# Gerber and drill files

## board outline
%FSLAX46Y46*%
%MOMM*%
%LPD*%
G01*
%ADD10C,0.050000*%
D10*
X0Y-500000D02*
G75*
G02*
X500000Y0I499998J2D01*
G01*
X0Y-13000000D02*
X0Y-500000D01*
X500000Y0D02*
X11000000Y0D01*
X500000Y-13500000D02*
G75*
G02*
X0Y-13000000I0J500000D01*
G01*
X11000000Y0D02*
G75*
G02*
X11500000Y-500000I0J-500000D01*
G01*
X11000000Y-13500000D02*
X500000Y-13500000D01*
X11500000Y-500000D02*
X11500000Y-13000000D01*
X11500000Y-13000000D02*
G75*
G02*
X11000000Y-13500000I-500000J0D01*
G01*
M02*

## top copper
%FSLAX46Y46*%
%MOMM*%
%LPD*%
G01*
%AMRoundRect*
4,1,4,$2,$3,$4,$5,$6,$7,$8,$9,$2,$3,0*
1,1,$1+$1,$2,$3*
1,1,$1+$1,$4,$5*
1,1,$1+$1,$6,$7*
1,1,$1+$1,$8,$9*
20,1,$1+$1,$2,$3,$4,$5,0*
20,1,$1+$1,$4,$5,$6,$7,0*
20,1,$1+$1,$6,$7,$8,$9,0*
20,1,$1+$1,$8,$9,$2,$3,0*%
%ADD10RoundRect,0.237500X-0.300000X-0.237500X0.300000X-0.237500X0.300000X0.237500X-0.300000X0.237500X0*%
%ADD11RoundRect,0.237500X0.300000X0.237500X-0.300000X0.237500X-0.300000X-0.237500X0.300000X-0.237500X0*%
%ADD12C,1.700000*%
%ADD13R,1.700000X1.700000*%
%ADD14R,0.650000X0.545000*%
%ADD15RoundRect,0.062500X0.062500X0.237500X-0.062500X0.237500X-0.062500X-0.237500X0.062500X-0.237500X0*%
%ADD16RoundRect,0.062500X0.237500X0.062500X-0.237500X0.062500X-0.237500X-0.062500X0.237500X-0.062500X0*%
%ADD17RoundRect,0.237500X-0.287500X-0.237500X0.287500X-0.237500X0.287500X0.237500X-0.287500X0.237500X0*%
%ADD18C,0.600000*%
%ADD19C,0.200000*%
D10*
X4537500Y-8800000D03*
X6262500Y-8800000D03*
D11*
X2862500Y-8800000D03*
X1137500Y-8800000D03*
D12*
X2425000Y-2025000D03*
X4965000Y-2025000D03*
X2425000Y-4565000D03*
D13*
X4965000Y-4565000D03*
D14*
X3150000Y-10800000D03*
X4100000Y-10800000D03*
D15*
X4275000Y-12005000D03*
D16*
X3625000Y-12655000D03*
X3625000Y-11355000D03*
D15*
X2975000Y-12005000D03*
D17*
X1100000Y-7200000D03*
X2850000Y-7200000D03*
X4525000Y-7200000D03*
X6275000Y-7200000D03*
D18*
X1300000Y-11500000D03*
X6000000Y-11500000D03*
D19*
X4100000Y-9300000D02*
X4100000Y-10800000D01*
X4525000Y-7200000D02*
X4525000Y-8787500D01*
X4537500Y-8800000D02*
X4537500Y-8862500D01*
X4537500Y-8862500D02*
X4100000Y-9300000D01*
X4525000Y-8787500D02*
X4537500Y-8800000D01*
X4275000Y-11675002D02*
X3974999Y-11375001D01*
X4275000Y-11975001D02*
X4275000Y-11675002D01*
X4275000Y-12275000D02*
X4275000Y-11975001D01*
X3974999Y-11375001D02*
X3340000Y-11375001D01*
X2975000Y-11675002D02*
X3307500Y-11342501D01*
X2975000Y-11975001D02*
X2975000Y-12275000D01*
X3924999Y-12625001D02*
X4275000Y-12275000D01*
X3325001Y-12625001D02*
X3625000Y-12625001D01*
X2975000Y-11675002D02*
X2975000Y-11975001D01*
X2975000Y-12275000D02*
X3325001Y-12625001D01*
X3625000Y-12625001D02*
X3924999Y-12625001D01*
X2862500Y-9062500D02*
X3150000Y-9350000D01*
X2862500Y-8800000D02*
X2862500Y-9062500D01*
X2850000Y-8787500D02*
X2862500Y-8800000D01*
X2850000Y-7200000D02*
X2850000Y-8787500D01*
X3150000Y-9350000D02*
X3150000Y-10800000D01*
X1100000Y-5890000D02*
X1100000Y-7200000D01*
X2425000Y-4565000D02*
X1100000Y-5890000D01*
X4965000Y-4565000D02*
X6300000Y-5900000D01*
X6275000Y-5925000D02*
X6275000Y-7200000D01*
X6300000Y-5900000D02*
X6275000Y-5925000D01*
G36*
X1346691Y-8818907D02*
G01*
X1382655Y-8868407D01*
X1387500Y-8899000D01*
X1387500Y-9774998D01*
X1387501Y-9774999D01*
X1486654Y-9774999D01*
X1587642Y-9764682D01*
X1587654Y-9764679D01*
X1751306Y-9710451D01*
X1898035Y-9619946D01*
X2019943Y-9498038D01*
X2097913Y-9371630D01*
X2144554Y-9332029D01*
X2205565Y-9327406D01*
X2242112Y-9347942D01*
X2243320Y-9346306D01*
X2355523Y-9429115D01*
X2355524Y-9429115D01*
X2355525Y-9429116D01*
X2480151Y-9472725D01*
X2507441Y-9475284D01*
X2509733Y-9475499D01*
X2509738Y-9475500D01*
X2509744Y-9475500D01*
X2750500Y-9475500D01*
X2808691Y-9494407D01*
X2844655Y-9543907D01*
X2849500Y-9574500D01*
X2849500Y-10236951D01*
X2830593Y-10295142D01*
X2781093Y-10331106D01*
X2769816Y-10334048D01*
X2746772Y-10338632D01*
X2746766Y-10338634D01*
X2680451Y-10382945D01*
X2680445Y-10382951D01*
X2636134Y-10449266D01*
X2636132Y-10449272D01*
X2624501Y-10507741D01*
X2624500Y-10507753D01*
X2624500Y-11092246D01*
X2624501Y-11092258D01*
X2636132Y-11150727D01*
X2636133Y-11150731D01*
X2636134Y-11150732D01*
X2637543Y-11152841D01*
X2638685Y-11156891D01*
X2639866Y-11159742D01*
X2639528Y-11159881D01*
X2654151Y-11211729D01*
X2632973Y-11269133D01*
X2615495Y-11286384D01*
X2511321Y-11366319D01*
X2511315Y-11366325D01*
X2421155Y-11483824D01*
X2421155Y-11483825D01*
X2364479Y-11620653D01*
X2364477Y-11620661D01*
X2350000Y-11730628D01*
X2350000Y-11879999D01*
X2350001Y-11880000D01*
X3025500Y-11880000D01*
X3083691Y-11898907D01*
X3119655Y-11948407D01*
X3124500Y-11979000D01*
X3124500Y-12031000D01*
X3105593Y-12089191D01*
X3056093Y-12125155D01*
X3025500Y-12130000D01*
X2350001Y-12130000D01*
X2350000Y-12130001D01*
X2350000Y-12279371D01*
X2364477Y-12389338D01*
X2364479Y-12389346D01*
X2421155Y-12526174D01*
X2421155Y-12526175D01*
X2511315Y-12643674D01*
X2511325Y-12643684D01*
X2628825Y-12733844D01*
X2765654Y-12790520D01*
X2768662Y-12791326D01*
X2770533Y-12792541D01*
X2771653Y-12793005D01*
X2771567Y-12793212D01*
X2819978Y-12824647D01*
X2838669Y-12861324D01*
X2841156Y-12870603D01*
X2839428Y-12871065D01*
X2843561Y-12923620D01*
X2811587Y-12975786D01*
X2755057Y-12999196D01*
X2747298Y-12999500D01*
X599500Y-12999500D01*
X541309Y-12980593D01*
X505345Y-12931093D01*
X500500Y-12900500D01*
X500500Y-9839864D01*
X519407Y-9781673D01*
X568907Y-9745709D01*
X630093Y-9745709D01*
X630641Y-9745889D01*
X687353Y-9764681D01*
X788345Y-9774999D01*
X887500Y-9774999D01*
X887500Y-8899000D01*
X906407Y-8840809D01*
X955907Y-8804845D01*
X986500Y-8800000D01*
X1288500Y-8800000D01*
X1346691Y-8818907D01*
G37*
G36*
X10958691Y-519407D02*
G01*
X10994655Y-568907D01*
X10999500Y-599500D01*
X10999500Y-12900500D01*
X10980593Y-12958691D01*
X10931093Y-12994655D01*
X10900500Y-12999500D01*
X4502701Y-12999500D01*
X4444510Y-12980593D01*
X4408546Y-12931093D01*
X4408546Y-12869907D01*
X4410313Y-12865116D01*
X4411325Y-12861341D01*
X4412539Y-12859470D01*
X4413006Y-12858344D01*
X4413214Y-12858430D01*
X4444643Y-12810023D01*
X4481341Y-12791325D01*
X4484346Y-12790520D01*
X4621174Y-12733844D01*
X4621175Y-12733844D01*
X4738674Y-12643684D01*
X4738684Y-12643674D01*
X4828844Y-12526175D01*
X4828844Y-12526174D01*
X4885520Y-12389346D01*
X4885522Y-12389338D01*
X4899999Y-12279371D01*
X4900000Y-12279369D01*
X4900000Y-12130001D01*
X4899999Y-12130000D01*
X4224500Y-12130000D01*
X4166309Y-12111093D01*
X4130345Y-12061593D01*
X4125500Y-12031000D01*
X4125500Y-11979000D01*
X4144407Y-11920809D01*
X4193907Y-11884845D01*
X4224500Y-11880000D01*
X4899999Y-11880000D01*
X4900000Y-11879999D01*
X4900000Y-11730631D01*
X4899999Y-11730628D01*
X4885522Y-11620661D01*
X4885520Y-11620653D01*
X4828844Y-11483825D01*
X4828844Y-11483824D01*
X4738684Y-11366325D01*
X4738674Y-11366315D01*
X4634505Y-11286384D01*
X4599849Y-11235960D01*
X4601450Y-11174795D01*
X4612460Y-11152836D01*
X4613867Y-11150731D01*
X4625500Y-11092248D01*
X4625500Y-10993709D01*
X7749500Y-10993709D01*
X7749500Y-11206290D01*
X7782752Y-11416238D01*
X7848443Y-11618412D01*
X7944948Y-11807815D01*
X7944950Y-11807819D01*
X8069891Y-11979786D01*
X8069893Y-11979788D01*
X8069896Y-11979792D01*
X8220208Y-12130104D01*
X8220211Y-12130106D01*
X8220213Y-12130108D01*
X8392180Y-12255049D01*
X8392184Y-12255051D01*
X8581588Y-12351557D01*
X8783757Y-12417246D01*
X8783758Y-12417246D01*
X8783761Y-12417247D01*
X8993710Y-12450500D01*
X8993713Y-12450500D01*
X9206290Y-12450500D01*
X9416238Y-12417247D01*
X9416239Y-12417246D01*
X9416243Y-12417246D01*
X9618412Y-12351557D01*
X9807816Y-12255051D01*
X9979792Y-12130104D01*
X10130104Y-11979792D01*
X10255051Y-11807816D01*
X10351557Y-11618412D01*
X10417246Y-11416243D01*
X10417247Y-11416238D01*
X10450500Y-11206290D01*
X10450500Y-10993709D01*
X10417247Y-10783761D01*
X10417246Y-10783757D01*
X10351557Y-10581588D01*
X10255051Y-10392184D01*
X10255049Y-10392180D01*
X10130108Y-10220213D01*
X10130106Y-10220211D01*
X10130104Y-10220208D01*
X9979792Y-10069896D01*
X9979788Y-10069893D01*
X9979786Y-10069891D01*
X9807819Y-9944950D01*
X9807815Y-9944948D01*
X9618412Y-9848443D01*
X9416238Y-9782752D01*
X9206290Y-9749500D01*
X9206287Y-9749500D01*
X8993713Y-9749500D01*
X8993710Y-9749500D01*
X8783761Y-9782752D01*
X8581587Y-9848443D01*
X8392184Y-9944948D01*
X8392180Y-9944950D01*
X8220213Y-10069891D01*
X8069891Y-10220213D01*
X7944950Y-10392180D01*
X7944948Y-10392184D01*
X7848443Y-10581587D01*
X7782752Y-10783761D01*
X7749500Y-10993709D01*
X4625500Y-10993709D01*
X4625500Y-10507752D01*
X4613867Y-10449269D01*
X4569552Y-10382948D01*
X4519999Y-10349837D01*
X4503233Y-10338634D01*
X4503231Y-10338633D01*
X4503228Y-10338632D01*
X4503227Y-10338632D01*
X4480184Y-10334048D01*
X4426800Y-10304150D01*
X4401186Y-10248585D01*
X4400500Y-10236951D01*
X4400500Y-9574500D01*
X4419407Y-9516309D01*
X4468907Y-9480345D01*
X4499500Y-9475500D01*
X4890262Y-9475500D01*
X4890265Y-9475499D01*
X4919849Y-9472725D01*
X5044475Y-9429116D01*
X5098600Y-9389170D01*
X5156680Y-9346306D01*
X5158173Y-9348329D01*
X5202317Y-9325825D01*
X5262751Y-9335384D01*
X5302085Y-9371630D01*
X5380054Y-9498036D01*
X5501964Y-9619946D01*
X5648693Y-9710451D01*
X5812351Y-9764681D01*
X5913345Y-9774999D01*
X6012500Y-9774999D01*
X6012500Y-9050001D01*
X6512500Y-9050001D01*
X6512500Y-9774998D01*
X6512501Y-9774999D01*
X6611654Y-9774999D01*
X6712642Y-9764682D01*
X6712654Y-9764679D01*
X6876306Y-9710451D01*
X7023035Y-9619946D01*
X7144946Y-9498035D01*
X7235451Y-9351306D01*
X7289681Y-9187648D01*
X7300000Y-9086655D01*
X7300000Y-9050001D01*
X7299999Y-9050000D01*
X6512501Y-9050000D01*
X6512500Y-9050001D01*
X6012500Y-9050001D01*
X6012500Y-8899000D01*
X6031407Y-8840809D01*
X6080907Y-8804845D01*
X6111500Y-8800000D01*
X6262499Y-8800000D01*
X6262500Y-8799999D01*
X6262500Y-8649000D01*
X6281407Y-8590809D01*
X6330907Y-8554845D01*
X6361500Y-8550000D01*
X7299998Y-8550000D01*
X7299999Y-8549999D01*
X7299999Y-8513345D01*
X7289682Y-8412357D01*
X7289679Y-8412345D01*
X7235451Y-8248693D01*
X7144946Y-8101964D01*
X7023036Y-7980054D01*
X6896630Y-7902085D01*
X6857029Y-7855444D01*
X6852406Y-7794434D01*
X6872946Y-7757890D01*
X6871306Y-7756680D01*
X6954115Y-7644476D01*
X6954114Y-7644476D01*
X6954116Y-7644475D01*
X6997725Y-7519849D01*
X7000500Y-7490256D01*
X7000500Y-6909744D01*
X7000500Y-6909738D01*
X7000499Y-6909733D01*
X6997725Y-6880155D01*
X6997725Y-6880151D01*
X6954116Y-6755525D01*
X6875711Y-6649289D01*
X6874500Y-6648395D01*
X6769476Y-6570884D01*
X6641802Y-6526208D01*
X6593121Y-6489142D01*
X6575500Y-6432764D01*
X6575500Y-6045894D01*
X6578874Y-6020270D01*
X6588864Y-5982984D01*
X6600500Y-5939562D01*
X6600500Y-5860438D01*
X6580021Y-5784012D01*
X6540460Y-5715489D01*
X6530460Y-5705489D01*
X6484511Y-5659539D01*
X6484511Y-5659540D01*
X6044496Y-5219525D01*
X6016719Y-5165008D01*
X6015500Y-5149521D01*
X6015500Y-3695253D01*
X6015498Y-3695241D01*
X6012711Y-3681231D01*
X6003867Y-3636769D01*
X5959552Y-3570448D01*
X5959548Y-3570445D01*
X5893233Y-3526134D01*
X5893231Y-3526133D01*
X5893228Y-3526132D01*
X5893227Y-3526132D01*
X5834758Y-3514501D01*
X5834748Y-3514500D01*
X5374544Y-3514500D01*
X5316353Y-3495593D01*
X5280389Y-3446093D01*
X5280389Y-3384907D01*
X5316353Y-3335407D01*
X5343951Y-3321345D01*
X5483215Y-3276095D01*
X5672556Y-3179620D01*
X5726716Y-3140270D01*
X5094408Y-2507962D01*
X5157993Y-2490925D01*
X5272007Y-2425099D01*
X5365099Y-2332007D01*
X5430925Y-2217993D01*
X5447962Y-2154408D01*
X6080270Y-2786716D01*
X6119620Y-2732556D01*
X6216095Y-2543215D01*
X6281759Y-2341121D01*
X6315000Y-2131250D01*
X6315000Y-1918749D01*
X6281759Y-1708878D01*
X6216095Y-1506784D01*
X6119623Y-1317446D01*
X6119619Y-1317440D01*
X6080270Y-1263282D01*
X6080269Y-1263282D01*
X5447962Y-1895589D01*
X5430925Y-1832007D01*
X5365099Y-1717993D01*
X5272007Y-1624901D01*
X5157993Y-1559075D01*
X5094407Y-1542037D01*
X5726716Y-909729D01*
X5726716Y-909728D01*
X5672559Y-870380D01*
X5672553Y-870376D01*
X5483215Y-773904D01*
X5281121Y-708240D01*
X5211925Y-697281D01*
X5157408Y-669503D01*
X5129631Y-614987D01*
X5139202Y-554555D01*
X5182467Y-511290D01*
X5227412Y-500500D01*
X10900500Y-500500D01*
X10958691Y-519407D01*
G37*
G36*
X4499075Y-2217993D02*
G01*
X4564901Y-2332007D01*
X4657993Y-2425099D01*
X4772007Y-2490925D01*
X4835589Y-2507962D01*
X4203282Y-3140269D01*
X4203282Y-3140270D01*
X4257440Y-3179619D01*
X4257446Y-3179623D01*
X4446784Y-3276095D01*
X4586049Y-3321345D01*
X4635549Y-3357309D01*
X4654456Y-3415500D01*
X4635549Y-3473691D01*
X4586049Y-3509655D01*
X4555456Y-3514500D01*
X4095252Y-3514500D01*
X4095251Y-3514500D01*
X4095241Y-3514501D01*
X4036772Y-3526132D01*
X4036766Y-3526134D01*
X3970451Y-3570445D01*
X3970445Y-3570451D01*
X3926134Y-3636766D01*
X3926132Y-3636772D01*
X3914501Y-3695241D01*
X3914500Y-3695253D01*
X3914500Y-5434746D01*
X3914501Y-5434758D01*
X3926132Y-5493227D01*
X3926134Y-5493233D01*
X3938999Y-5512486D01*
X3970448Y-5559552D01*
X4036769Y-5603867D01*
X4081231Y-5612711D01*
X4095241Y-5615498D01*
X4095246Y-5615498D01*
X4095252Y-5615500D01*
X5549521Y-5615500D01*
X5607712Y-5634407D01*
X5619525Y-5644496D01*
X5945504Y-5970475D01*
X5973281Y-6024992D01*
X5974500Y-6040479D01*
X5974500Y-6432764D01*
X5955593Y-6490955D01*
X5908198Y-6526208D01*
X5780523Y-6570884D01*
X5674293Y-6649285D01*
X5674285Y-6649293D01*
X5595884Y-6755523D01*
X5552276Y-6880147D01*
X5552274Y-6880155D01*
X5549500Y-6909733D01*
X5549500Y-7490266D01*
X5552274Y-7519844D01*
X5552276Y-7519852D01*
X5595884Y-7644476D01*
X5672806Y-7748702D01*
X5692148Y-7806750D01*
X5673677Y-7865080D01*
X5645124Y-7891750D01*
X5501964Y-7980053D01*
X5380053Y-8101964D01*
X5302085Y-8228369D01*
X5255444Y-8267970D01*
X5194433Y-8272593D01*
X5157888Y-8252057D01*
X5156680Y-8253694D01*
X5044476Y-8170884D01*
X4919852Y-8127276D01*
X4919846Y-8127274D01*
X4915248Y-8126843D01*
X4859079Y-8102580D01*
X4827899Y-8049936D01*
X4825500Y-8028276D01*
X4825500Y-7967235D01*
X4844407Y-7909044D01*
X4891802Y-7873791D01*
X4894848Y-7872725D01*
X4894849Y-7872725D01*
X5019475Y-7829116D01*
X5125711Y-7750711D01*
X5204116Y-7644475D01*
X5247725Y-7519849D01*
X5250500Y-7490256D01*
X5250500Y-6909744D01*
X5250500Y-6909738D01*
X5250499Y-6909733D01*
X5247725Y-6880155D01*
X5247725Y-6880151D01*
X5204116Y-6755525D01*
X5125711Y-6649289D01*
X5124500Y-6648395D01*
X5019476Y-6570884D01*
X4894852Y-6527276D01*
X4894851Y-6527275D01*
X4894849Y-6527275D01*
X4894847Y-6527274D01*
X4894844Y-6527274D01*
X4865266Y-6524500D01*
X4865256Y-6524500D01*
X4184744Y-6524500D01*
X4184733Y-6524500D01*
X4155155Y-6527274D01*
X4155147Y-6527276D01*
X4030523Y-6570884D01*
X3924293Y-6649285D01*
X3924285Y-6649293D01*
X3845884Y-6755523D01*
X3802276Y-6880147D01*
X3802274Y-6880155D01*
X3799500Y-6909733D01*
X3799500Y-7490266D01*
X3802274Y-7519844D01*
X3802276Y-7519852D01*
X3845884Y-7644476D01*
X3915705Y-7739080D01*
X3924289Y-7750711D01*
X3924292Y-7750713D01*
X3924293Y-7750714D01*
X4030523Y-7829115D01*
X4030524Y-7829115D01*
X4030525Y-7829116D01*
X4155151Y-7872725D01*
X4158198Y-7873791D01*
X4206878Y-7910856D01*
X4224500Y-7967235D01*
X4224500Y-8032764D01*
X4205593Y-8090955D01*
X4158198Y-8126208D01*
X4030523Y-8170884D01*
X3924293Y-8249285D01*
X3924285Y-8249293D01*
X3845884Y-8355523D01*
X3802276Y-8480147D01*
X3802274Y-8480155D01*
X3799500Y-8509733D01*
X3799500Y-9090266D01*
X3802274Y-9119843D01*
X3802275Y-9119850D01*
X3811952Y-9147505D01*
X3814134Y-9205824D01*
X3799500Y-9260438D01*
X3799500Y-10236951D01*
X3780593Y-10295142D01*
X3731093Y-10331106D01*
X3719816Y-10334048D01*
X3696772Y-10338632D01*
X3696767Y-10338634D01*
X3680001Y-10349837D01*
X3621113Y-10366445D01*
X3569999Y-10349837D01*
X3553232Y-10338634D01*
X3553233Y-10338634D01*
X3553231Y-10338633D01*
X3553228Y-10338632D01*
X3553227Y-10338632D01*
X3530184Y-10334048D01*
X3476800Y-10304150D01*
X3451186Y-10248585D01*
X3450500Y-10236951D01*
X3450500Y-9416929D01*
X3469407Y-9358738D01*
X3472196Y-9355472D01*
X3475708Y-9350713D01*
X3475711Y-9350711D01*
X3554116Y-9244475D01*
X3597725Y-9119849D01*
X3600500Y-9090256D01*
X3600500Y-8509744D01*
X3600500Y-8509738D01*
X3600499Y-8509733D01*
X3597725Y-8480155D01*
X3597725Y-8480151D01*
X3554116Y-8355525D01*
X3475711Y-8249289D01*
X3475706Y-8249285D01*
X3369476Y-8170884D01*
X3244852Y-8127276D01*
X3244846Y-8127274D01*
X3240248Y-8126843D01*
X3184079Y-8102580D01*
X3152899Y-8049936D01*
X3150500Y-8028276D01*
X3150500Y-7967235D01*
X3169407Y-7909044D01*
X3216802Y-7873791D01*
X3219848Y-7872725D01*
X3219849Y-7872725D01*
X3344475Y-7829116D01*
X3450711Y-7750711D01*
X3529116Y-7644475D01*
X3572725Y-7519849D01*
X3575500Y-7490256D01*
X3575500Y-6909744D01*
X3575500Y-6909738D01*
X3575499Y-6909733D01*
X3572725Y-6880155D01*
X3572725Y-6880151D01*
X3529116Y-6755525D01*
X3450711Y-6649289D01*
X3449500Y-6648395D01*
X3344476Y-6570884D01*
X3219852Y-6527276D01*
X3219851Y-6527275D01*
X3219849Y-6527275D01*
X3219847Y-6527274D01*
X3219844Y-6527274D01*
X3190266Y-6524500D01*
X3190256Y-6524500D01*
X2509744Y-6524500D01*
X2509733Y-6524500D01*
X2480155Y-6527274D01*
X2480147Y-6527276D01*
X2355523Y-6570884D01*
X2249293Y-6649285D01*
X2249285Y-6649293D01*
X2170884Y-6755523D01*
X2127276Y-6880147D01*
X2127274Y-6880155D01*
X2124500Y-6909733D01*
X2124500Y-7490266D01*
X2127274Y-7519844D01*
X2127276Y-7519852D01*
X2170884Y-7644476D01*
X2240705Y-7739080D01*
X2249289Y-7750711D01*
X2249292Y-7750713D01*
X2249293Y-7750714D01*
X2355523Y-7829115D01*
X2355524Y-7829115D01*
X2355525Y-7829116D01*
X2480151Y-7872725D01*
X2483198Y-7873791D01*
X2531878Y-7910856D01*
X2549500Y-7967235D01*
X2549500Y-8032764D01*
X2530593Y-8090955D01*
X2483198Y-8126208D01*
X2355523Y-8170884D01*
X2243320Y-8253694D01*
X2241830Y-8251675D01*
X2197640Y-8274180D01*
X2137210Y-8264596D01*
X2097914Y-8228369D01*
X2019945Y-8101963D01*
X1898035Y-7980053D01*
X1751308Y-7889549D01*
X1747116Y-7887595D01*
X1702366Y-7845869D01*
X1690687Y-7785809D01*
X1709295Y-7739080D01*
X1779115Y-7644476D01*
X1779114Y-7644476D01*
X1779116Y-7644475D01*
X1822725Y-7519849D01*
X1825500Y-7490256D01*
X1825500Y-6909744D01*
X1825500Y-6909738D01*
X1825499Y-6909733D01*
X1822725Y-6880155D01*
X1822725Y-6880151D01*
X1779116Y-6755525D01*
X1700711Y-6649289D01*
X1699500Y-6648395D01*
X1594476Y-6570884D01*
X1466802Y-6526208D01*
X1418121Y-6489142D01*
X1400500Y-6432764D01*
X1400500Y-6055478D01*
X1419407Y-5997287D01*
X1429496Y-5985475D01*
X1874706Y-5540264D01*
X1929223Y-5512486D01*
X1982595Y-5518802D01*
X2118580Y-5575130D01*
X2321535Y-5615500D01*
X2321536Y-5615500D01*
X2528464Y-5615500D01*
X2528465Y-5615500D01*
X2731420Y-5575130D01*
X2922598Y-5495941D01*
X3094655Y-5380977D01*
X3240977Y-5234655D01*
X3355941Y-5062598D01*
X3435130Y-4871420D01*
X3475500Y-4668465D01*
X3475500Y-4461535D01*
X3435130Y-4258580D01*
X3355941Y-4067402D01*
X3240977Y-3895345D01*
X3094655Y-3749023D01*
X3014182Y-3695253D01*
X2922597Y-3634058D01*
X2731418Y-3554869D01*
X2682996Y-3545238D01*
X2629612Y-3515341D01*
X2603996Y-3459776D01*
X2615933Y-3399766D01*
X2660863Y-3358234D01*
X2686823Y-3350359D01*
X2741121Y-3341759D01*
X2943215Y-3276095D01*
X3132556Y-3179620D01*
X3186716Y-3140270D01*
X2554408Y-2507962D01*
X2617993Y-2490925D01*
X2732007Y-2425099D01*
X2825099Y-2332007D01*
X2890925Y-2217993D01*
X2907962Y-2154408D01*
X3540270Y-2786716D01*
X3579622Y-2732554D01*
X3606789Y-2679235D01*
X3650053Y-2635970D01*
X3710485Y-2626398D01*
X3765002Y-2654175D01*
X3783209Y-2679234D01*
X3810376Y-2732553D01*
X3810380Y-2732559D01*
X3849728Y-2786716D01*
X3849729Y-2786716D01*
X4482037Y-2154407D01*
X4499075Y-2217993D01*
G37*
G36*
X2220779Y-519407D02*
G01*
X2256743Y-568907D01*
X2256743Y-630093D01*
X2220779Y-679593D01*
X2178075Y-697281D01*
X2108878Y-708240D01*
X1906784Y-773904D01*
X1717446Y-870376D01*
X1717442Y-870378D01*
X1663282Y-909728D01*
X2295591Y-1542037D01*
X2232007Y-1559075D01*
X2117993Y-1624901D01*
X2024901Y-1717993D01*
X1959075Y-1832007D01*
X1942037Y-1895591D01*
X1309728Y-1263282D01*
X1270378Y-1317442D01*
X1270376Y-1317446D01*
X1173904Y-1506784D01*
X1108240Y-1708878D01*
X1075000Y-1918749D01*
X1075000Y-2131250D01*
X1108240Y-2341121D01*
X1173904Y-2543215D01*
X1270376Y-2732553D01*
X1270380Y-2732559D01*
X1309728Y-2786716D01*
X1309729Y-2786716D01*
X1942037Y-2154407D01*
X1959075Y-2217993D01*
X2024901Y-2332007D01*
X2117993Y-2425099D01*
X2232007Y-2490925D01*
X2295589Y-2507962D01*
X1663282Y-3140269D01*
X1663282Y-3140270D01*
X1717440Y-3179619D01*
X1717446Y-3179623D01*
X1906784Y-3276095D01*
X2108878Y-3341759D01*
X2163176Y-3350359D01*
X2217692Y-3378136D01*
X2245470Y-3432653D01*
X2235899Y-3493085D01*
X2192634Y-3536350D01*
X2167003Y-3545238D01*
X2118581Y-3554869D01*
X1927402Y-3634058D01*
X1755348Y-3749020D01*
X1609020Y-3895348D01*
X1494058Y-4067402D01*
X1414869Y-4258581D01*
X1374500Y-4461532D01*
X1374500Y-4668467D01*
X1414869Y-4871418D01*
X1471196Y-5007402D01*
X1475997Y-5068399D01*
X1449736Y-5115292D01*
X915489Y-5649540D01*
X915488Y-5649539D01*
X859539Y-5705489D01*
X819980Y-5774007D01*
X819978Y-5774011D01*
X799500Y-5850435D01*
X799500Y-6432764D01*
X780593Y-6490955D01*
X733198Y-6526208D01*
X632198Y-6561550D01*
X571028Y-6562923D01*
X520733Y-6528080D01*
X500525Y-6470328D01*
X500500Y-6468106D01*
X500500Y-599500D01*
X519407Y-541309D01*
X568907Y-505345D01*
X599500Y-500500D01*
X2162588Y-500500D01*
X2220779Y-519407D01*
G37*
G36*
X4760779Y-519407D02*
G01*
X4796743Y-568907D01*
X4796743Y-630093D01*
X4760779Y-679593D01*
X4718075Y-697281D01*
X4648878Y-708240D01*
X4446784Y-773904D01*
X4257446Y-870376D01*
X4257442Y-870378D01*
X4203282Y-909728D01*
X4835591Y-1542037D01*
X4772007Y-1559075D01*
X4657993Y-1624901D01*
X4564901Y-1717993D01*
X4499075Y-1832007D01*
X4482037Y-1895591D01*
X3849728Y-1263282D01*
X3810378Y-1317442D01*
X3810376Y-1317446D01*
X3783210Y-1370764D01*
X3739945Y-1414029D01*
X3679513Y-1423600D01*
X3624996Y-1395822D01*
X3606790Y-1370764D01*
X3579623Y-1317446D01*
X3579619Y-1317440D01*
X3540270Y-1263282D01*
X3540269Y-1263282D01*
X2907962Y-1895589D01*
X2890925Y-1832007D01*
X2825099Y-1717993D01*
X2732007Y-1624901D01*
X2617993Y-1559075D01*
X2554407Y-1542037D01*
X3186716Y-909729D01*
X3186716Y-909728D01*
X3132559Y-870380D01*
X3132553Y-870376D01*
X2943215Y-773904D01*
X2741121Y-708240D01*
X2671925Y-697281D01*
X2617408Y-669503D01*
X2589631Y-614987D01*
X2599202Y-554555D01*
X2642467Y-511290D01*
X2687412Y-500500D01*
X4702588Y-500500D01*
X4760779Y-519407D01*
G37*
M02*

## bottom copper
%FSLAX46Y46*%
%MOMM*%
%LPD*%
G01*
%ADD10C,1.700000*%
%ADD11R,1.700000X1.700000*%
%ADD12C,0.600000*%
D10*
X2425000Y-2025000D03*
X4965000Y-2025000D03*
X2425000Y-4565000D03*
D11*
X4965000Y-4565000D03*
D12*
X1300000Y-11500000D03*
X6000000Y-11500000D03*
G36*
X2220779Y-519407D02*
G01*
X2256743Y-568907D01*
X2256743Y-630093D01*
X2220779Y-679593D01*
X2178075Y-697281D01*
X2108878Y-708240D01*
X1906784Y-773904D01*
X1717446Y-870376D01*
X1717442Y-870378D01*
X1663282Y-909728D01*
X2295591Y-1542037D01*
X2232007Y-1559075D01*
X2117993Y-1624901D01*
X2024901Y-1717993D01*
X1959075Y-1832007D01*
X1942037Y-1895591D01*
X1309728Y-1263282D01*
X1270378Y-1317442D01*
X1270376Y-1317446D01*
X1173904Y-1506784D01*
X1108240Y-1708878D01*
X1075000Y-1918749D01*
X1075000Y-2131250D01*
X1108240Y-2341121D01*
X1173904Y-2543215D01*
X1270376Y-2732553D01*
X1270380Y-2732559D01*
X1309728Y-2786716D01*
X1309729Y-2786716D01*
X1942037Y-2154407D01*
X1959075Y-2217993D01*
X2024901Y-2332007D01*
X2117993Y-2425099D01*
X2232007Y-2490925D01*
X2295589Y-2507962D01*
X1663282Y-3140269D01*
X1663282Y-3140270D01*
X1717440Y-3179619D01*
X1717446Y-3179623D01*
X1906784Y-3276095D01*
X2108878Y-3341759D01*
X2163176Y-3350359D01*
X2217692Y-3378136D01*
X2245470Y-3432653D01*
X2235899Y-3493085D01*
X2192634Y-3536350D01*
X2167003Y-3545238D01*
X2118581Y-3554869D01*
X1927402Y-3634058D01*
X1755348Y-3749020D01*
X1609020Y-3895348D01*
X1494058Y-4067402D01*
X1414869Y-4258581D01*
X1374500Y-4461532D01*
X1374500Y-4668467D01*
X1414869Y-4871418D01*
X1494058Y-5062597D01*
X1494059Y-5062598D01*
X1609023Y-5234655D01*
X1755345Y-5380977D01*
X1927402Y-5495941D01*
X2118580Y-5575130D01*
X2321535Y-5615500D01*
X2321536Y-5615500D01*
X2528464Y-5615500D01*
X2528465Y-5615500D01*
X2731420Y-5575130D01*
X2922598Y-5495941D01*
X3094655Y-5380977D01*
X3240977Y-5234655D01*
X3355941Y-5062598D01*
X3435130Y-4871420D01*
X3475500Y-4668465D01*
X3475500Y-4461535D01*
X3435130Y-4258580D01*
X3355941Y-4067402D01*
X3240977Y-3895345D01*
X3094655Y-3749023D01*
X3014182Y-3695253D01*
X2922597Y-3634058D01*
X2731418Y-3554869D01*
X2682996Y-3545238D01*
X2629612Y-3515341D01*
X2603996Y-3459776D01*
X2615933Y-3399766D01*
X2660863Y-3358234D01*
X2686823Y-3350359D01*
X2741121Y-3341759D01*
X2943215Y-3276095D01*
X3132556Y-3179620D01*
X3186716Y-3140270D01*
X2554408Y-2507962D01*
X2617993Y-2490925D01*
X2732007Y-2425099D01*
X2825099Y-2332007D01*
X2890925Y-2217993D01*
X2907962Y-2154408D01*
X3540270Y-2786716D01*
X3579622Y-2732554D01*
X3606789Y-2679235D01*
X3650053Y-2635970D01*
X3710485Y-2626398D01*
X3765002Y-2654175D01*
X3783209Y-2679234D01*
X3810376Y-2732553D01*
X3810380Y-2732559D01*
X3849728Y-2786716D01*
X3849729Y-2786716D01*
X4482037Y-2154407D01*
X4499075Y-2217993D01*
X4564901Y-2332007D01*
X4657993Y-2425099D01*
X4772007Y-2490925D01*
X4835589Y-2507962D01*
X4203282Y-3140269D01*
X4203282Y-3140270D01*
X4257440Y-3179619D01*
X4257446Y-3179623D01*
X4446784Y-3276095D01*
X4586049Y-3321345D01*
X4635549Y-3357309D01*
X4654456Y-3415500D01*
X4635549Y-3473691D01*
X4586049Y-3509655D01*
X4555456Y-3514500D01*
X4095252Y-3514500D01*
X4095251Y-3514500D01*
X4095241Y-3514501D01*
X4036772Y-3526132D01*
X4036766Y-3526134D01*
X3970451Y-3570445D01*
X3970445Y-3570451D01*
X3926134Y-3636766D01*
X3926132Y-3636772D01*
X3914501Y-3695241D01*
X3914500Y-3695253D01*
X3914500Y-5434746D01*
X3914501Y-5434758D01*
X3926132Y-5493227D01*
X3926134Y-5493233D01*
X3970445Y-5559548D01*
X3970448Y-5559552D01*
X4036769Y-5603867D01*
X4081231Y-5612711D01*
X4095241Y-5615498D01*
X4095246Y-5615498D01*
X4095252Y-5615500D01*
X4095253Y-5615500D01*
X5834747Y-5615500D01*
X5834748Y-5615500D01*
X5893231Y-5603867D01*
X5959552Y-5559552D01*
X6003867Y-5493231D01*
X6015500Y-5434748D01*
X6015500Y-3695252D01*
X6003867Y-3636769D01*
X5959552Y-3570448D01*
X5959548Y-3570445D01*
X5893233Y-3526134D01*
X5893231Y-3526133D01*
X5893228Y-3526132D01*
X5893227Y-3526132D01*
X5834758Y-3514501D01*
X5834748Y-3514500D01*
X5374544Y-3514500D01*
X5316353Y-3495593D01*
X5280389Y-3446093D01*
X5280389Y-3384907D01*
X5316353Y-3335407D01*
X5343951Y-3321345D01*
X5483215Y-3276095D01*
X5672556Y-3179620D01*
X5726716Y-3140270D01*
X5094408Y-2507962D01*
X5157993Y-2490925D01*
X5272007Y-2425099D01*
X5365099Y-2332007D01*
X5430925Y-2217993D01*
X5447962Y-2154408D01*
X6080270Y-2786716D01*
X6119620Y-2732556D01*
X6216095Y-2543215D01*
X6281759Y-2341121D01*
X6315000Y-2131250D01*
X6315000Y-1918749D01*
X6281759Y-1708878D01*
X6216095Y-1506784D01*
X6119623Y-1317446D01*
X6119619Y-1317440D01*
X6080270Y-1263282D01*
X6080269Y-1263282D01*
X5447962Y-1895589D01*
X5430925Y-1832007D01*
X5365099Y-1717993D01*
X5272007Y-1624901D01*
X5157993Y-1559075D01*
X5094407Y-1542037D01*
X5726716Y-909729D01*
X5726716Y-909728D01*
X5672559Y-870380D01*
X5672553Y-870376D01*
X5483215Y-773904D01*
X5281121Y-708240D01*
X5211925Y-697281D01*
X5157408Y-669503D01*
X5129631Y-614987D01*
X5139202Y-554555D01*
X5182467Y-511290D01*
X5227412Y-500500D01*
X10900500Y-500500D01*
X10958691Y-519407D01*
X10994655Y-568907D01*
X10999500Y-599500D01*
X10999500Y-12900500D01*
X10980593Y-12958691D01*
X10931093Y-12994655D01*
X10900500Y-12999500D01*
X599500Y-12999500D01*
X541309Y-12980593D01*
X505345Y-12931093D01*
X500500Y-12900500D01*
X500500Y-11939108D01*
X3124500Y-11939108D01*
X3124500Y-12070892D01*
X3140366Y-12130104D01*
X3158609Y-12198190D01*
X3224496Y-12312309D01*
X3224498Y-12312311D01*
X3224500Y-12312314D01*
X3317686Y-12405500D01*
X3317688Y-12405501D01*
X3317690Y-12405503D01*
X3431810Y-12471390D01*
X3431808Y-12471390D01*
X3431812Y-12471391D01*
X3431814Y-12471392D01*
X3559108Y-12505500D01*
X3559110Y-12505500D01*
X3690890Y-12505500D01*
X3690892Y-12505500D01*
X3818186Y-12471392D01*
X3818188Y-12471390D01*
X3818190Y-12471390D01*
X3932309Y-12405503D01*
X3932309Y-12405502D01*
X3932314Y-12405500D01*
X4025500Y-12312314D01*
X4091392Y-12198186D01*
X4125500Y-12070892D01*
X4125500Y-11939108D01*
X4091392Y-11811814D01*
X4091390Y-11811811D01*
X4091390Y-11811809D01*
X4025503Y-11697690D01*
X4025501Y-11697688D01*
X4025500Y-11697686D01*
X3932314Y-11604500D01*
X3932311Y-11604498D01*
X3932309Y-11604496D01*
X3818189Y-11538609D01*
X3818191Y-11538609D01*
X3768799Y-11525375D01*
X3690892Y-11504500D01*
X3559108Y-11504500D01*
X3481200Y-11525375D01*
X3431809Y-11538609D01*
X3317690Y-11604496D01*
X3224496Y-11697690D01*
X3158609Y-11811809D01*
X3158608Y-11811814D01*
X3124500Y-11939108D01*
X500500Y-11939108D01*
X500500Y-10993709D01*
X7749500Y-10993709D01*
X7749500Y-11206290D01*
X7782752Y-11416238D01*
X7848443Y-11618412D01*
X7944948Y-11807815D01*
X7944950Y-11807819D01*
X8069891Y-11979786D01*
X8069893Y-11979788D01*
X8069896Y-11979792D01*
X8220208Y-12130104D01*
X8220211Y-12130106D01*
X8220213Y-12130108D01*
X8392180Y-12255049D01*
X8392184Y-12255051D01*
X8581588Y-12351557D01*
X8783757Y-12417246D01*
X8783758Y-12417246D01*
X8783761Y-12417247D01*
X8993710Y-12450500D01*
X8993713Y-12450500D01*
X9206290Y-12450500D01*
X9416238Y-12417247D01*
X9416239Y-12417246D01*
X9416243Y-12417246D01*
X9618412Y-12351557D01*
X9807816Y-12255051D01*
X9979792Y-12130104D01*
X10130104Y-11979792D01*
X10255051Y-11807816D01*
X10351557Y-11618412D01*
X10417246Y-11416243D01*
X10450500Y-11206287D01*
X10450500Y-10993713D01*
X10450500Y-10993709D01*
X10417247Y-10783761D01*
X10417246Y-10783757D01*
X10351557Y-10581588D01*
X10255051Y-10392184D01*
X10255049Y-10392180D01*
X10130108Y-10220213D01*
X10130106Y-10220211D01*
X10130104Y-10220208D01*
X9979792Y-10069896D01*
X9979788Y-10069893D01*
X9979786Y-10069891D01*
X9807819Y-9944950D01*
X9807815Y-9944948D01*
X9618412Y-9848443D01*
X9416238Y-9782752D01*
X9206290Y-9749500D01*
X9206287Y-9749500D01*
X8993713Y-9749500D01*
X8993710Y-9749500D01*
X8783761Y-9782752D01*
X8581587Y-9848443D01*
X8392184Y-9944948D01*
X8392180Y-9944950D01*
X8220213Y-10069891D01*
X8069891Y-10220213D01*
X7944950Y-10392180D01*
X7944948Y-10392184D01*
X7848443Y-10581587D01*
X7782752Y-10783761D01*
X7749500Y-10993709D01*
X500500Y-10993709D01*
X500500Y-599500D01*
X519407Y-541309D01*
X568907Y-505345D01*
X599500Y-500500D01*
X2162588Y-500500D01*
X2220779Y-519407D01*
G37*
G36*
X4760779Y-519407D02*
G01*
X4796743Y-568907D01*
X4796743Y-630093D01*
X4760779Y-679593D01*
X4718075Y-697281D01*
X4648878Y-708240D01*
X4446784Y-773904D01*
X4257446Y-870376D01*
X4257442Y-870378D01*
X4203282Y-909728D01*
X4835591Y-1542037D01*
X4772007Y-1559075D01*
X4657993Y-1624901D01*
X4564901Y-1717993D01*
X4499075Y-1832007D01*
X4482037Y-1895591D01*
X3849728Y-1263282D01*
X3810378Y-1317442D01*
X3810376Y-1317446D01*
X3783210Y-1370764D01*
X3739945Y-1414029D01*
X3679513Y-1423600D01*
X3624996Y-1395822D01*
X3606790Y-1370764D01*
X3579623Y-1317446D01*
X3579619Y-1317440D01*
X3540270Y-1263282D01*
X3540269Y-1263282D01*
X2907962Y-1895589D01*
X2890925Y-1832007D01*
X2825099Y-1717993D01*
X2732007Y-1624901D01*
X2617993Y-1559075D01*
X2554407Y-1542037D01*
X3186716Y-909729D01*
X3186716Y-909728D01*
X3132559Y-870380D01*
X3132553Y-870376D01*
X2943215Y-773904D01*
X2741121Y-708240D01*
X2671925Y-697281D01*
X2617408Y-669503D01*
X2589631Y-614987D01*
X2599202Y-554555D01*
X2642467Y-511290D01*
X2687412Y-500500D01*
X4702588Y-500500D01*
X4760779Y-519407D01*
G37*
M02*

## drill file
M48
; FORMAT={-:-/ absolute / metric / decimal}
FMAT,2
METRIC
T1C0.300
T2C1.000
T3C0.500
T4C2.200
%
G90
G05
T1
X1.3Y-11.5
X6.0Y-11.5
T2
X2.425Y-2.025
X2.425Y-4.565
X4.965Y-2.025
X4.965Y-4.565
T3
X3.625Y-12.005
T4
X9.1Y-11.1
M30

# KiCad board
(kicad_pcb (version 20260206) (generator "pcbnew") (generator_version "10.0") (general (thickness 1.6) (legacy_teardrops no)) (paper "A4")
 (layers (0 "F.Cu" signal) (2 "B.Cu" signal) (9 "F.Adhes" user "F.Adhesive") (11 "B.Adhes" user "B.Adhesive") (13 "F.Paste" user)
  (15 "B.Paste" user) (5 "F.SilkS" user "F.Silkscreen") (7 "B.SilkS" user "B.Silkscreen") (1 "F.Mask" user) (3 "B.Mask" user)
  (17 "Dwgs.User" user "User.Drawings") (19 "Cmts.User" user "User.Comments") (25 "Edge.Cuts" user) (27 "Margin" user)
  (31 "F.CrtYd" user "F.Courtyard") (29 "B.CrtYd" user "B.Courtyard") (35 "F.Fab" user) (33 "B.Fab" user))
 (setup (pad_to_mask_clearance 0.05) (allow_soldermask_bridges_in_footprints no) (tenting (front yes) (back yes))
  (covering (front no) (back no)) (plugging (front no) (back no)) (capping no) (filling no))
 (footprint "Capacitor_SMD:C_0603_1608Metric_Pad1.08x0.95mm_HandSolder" (layer "F.Cu") (at 5.4 8.8)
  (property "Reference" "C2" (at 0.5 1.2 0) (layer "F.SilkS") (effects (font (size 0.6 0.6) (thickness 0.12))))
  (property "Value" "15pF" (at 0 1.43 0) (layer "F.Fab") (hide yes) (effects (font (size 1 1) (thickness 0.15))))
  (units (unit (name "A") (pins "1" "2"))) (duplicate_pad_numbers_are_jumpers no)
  (pad "1" smd roundrect (at -0.8625 0) (size 1.075 0.95) (layers "F.Cu" "F.Mask" "F.Paste") (roundrect_rratio 0.25) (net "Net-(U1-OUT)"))
  (pad "2" smd roundrect (at 0.8625 0) (size 1.075 0.95) (layers "F.Cu" "F.Mask" "F.Paste") (roundrect_rratio 0.25) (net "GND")))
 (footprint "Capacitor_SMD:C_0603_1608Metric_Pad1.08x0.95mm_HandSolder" (layer "F.Cu") (at 2 8.8 180)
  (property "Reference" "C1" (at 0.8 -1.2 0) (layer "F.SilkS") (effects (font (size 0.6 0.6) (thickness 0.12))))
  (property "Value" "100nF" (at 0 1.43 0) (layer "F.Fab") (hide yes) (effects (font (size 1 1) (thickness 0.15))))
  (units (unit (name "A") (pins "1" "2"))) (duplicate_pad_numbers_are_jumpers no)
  (pad "1" smd roundrect (at -0.8625 0 180) (size 1.075 0.95) (layers "F.Cu" "F.Mask" "F.Paste") (roundrect_rratio 0.25) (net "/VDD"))
  (pad "2" smd roundrect (at 0.8625 0 180) (size 1.075 0.95) (layers "F.Cu" "F.Mask" "F.Paste") (roundrect_rratio 0.25) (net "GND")))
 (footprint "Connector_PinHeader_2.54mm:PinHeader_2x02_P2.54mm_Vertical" (layer "F.Cu") (at 2.425 2.025)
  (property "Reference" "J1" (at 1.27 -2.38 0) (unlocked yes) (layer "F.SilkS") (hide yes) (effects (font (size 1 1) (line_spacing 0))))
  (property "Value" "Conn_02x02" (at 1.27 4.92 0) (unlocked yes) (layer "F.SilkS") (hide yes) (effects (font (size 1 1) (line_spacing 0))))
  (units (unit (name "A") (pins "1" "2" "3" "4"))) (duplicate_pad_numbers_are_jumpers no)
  (pad "1" thru_hole circle (at 0 0) (size 1.7 1.7) (drill 1) (layers "*.Cu" "*.Mask") (remove_unused_layers no) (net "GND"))
  (pad "2" thru_hole circle (at 2.54 0) (size 1.7 1.7) (drill 1) (layers "*.Cu" "*.Mask") (remove_unused_layers no) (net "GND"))
  (pad "3" thru_hole circle (at 0 2.54) (size 1.7 1.7) (drill 1) (layers "*.Cu" "*.Mask") (remove_unused_layers no) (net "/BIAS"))
  (pad "4" thru_hole rect (at 2.54 2.54) (size 1.7 1.7) (drill 1) (layers "*.Cu" "*.Mask") (remove_unused_layers no) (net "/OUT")))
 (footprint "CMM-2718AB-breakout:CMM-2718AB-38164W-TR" (layer "F.Cu") (at 3.625 12.005 180)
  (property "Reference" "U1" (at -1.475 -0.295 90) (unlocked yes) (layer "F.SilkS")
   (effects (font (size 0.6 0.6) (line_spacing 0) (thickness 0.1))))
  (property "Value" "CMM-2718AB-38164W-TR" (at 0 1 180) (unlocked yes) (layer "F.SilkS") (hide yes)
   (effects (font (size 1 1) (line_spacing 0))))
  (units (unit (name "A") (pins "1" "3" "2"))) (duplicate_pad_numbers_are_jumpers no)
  (pad "" np_thru_hole circle (at 0 0 180) (size 0.5 0.5) (drill 0.5) (layers "*.Cu" "*.Mask"))
  (pad "1" smd rect (at 0.475 1.205 180) (size 0.65 0.545) (layers "F.Cu" "F.Mask" "F.Paste") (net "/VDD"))
  (pad "2" smd rect (at -0.475 1.205 180) (size 0.65 0.545) (layers "F.Cu" "F.Mask" "F.Paste") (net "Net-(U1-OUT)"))
  (pad "3" smd roundrect (at -0.65 0 180) (size 0.25 0.6) (layers "F.Cu" "F.Mask" "F.Paste") (roundrect_rratio 0.25) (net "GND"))
  (pad "3" smd roundrect (at 0 -0.65 180) (size 0.6 0.25) (layers "F.Cu" "F.Mask" "F.Paste") (roundrect_rratio 0.25) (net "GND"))
  (pad "3" smd roundrect (at 0 0.65 180) (size 0.6 0.25) (layers "F.Cu" "F.Mask" "F.Paste") (roundrect_rratio 0.25) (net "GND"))
  (pad "3" smd roundrect (at 0.65 0 180) (size 0.25 0.6) (layers "F.Cu" "F.Mask" "F.Paste") (roundrect_rratio 0.25) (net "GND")))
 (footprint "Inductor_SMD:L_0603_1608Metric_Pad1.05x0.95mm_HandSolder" (layer "F.Cu") (at 1.975 7.2)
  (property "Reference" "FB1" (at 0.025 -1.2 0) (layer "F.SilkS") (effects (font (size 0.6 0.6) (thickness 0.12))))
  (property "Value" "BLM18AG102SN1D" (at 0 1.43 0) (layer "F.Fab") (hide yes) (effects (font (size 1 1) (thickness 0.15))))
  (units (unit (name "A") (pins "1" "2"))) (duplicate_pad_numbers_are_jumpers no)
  (pad "1" smd roundrect (at -0.875 0) (size 1.05 0.95) (layers "F.Cu" "F.Mask" "F.Paste") (roundrect_rratio 0.25) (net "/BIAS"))
  (pad "2" smd roundrect (at 0.875 0) (size 1.05 0.95) (layers "F.Cu" "F.Mask" "F.Paste") (roundrect_rratio 0.25) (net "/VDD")))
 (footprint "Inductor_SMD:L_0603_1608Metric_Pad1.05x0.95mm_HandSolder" (layer "F.Cu") (at 5.4 7.2)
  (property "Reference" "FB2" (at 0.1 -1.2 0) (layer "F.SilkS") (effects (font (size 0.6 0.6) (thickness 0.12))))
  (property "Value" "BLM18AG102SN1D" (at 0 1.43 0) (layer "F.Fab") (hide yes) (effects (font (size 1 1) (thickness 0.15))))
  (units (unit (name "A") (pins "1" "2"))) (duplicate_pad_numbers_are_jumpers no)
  (pad "1" smd roundrect (at -0.875 0) (size 1.05 0.95) (layers "F.Cu" "F.Mask" "F.Paste") (roundrect_rratio 0.25) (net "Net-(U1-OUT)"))
  (pad "2" smd roundrect (at 0.875 0) (size 1.05 0.95) (layers "F.Cu" "F.Mask" "F.Paste") (roundrect_rratio 0.25) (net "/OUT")))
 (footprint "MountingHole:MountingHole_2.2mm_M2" (layer "F.Cu") (at 9.1 11.1)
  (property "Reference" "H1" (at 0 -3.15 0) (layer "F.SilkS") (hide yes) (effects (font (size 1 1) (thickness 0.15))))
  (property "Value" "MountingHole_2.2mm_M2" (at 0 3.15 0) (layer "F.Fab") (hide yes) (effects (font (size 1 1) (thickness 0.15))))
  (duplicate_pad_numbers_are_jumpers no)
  (pad "" np_thru_hole circle (at 0 0) (size 2.2 2.2) (drill 2.2) (layers "*.Cu" "*.Mask")))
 (gr_arc (start 0 0.5) (mid 0.146446 0.146446) (end 0.5 0) (stroke (width 0.05) (type default)) (layer "Edge.Cuts"))
 (gr_line (start 0 13) (end 0 0.5) (stroke (width 0.05) (type default)) (layer "Edge.Cuts"))
 (gr_line (start 0.5 0) (end 11 0) (stroke (width 0.05) (type default)) (layer "Edge.Cuts"))
 (gr_arc (start 0.5 13.5) (mid 0.146446 13.353553) (end 0 13) (stroke (width 0.05) (type default)) (layer "Edge.Cuts"))
 (gr_arc (start 11 0) (mid 11.353553 0.146446) (end 11.5 0.5) (stroke (width 0.05) (type default)) (layer "Edge.Cuts"))
 (gr_line (start 11 13.5) (end 0.5 13.5) (stroke (width 0.05) (type default)) (layer "Edge.Cuts"))
 (gr_line (start 11.5 0.5) (end 11.5 13) (stroke (width 0.05) (type default)) (layer "Edge.Cuts"))
 (gr_arc (start 11.5 13) (mid 11.353553 13.353553) (end 11 13.5) (stroke (width 0.05) (type default)) (layer "Edge.Cuts"))
 (segment (start 4.1 9.3) (end 4.1 10.8) (width 0.2) (layer "F.Cu") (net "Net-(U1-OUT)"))
 (segment (start 4.525 7.2) (end 4.525 8.7875) (width 0.2) (layer "F.Cu") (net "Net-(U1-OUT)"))
 (segment (start 4.5375 8.8) (end 4.5375 8.8625) (width 0.2) (layer "F.Cu") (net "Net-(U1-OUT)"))
 (segment (start 4.5375 8.8625) (end 4.1 9.3) (width 0.2) (layer "F.Cu") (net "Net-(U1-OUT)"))
 (segment (start 4.525 8.7875) (end 4.5375 8.8) (width 0.2) (layer "F.Cu") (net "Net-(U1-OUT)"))
 (segment (start 4.275 11.675002) (end 3.974999 11.375001) (width 0.2) (layer "F.Cu") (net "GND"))
 (segment (start 4.275 11.975001) (end 4.275 11.675002) (width 0.2) (layer "F.Cu") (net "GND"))
 (segment (start 4.275 12.275) (end 4.275 11.975001) (width 0.2) (layer "F.Cu") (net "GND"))
 (segment (start 3.974999 11.375001) (end 3.34 11.375001) (width 0.2) (layer "F.Cu") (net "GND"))
 (segment (start 2.975 11.675002) (end 3.3075 11.342501) (width 0.2) (layer "F.Cu") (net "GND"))
 (segment (start 2.975 11.975001) (end 2.975 12.275) (width 0.2) (layer "F.Cu") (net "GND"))
 (segment (start 3.924999 12.625001) (end 4.275 12.275) (width 0.2) (layer "F.Cu") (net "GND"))
 (segment (start 3.325001 12.625001) (end 3.625 12.625001) (width 0.2) (layer "F.Cu") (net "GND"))
 (segment (start 2.975 11.675002) (end 2.975 11.975001) (width 0.2) (layer "F.Cu") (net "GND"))
 (segment (start 2.975 12.275) (end 3.325001 12.625001) (width 0.2) (layer "F.Cu") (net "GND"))
 (segment (start 3.625 12.625001) (end 3.924999 12.625001) (width 0.2) (layer "F.Cu") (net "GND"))
 (via (at 1.3 11.5) (size 0.6) (drill 0.3) (layers "F.Cu" "B.Cu") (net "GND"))
 (via (at 6 11.5) (size 0.6) (drill 0.3) (layers "F.Cu" "B.Cu") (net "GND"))
 (segment (start 2.8625 9.0625) (end 3.15 9.35) (width 0.2) (layer "F.Cu") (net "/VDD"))
 (segment (start 2.8625 8.8) (end 2.8625 9.0625) (width 0.2) (layer "F.Cu") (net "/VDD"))
 (segment (start 2.85 8.7875) (end 2.8625 8.8) (width 0.2) (layer "F.Cu") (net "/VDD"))
 (segment (start 2.85 7.2) (end 2.85 8.7875) (width 0.2) (layer "F.Cu") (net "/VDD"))
 (segment (start 3.15 9.35) (end 3.15 10.8) (width 0.2) (layer "F.Cu") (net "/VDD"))
 (segment (start 1.1 5.89) (end 1.1 7.2) (width 0.2) (layer "F.Cu") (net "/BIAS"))
 (segment (start 2.425 4.565) (end 1.1 5.89) (width 0.2) (layer "F.Cu") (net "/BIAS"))
 (segment (start 4.965 4.565) (end 6.3 5.9) (width 0.2) (layer "F.Cu") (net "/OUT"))
 (segment (start 6.275 5.925) (end 6.275 7.2) (width 0.2) (layer "F.Cu") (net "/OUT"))
 (segment (start 6.3 5.9) (end 6.275 5.925) (width 0.2) (layer "F.Cu") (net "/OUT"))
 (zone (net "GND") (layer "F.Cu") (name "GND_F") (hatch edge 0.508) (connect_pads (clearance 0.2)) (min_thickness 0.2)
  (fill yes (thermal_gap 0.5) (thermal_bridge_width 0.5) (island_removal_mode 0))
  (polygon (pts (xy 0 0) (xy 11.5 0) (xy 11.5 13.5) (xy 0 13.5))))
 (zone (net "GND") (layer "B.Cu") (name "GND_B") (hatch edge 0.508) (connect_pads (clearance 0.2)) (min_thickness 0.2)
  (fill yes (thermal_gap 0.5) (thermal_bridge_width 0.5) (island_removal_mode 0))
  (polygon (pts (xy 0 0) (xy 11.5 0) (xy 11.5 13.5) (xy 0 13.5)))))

